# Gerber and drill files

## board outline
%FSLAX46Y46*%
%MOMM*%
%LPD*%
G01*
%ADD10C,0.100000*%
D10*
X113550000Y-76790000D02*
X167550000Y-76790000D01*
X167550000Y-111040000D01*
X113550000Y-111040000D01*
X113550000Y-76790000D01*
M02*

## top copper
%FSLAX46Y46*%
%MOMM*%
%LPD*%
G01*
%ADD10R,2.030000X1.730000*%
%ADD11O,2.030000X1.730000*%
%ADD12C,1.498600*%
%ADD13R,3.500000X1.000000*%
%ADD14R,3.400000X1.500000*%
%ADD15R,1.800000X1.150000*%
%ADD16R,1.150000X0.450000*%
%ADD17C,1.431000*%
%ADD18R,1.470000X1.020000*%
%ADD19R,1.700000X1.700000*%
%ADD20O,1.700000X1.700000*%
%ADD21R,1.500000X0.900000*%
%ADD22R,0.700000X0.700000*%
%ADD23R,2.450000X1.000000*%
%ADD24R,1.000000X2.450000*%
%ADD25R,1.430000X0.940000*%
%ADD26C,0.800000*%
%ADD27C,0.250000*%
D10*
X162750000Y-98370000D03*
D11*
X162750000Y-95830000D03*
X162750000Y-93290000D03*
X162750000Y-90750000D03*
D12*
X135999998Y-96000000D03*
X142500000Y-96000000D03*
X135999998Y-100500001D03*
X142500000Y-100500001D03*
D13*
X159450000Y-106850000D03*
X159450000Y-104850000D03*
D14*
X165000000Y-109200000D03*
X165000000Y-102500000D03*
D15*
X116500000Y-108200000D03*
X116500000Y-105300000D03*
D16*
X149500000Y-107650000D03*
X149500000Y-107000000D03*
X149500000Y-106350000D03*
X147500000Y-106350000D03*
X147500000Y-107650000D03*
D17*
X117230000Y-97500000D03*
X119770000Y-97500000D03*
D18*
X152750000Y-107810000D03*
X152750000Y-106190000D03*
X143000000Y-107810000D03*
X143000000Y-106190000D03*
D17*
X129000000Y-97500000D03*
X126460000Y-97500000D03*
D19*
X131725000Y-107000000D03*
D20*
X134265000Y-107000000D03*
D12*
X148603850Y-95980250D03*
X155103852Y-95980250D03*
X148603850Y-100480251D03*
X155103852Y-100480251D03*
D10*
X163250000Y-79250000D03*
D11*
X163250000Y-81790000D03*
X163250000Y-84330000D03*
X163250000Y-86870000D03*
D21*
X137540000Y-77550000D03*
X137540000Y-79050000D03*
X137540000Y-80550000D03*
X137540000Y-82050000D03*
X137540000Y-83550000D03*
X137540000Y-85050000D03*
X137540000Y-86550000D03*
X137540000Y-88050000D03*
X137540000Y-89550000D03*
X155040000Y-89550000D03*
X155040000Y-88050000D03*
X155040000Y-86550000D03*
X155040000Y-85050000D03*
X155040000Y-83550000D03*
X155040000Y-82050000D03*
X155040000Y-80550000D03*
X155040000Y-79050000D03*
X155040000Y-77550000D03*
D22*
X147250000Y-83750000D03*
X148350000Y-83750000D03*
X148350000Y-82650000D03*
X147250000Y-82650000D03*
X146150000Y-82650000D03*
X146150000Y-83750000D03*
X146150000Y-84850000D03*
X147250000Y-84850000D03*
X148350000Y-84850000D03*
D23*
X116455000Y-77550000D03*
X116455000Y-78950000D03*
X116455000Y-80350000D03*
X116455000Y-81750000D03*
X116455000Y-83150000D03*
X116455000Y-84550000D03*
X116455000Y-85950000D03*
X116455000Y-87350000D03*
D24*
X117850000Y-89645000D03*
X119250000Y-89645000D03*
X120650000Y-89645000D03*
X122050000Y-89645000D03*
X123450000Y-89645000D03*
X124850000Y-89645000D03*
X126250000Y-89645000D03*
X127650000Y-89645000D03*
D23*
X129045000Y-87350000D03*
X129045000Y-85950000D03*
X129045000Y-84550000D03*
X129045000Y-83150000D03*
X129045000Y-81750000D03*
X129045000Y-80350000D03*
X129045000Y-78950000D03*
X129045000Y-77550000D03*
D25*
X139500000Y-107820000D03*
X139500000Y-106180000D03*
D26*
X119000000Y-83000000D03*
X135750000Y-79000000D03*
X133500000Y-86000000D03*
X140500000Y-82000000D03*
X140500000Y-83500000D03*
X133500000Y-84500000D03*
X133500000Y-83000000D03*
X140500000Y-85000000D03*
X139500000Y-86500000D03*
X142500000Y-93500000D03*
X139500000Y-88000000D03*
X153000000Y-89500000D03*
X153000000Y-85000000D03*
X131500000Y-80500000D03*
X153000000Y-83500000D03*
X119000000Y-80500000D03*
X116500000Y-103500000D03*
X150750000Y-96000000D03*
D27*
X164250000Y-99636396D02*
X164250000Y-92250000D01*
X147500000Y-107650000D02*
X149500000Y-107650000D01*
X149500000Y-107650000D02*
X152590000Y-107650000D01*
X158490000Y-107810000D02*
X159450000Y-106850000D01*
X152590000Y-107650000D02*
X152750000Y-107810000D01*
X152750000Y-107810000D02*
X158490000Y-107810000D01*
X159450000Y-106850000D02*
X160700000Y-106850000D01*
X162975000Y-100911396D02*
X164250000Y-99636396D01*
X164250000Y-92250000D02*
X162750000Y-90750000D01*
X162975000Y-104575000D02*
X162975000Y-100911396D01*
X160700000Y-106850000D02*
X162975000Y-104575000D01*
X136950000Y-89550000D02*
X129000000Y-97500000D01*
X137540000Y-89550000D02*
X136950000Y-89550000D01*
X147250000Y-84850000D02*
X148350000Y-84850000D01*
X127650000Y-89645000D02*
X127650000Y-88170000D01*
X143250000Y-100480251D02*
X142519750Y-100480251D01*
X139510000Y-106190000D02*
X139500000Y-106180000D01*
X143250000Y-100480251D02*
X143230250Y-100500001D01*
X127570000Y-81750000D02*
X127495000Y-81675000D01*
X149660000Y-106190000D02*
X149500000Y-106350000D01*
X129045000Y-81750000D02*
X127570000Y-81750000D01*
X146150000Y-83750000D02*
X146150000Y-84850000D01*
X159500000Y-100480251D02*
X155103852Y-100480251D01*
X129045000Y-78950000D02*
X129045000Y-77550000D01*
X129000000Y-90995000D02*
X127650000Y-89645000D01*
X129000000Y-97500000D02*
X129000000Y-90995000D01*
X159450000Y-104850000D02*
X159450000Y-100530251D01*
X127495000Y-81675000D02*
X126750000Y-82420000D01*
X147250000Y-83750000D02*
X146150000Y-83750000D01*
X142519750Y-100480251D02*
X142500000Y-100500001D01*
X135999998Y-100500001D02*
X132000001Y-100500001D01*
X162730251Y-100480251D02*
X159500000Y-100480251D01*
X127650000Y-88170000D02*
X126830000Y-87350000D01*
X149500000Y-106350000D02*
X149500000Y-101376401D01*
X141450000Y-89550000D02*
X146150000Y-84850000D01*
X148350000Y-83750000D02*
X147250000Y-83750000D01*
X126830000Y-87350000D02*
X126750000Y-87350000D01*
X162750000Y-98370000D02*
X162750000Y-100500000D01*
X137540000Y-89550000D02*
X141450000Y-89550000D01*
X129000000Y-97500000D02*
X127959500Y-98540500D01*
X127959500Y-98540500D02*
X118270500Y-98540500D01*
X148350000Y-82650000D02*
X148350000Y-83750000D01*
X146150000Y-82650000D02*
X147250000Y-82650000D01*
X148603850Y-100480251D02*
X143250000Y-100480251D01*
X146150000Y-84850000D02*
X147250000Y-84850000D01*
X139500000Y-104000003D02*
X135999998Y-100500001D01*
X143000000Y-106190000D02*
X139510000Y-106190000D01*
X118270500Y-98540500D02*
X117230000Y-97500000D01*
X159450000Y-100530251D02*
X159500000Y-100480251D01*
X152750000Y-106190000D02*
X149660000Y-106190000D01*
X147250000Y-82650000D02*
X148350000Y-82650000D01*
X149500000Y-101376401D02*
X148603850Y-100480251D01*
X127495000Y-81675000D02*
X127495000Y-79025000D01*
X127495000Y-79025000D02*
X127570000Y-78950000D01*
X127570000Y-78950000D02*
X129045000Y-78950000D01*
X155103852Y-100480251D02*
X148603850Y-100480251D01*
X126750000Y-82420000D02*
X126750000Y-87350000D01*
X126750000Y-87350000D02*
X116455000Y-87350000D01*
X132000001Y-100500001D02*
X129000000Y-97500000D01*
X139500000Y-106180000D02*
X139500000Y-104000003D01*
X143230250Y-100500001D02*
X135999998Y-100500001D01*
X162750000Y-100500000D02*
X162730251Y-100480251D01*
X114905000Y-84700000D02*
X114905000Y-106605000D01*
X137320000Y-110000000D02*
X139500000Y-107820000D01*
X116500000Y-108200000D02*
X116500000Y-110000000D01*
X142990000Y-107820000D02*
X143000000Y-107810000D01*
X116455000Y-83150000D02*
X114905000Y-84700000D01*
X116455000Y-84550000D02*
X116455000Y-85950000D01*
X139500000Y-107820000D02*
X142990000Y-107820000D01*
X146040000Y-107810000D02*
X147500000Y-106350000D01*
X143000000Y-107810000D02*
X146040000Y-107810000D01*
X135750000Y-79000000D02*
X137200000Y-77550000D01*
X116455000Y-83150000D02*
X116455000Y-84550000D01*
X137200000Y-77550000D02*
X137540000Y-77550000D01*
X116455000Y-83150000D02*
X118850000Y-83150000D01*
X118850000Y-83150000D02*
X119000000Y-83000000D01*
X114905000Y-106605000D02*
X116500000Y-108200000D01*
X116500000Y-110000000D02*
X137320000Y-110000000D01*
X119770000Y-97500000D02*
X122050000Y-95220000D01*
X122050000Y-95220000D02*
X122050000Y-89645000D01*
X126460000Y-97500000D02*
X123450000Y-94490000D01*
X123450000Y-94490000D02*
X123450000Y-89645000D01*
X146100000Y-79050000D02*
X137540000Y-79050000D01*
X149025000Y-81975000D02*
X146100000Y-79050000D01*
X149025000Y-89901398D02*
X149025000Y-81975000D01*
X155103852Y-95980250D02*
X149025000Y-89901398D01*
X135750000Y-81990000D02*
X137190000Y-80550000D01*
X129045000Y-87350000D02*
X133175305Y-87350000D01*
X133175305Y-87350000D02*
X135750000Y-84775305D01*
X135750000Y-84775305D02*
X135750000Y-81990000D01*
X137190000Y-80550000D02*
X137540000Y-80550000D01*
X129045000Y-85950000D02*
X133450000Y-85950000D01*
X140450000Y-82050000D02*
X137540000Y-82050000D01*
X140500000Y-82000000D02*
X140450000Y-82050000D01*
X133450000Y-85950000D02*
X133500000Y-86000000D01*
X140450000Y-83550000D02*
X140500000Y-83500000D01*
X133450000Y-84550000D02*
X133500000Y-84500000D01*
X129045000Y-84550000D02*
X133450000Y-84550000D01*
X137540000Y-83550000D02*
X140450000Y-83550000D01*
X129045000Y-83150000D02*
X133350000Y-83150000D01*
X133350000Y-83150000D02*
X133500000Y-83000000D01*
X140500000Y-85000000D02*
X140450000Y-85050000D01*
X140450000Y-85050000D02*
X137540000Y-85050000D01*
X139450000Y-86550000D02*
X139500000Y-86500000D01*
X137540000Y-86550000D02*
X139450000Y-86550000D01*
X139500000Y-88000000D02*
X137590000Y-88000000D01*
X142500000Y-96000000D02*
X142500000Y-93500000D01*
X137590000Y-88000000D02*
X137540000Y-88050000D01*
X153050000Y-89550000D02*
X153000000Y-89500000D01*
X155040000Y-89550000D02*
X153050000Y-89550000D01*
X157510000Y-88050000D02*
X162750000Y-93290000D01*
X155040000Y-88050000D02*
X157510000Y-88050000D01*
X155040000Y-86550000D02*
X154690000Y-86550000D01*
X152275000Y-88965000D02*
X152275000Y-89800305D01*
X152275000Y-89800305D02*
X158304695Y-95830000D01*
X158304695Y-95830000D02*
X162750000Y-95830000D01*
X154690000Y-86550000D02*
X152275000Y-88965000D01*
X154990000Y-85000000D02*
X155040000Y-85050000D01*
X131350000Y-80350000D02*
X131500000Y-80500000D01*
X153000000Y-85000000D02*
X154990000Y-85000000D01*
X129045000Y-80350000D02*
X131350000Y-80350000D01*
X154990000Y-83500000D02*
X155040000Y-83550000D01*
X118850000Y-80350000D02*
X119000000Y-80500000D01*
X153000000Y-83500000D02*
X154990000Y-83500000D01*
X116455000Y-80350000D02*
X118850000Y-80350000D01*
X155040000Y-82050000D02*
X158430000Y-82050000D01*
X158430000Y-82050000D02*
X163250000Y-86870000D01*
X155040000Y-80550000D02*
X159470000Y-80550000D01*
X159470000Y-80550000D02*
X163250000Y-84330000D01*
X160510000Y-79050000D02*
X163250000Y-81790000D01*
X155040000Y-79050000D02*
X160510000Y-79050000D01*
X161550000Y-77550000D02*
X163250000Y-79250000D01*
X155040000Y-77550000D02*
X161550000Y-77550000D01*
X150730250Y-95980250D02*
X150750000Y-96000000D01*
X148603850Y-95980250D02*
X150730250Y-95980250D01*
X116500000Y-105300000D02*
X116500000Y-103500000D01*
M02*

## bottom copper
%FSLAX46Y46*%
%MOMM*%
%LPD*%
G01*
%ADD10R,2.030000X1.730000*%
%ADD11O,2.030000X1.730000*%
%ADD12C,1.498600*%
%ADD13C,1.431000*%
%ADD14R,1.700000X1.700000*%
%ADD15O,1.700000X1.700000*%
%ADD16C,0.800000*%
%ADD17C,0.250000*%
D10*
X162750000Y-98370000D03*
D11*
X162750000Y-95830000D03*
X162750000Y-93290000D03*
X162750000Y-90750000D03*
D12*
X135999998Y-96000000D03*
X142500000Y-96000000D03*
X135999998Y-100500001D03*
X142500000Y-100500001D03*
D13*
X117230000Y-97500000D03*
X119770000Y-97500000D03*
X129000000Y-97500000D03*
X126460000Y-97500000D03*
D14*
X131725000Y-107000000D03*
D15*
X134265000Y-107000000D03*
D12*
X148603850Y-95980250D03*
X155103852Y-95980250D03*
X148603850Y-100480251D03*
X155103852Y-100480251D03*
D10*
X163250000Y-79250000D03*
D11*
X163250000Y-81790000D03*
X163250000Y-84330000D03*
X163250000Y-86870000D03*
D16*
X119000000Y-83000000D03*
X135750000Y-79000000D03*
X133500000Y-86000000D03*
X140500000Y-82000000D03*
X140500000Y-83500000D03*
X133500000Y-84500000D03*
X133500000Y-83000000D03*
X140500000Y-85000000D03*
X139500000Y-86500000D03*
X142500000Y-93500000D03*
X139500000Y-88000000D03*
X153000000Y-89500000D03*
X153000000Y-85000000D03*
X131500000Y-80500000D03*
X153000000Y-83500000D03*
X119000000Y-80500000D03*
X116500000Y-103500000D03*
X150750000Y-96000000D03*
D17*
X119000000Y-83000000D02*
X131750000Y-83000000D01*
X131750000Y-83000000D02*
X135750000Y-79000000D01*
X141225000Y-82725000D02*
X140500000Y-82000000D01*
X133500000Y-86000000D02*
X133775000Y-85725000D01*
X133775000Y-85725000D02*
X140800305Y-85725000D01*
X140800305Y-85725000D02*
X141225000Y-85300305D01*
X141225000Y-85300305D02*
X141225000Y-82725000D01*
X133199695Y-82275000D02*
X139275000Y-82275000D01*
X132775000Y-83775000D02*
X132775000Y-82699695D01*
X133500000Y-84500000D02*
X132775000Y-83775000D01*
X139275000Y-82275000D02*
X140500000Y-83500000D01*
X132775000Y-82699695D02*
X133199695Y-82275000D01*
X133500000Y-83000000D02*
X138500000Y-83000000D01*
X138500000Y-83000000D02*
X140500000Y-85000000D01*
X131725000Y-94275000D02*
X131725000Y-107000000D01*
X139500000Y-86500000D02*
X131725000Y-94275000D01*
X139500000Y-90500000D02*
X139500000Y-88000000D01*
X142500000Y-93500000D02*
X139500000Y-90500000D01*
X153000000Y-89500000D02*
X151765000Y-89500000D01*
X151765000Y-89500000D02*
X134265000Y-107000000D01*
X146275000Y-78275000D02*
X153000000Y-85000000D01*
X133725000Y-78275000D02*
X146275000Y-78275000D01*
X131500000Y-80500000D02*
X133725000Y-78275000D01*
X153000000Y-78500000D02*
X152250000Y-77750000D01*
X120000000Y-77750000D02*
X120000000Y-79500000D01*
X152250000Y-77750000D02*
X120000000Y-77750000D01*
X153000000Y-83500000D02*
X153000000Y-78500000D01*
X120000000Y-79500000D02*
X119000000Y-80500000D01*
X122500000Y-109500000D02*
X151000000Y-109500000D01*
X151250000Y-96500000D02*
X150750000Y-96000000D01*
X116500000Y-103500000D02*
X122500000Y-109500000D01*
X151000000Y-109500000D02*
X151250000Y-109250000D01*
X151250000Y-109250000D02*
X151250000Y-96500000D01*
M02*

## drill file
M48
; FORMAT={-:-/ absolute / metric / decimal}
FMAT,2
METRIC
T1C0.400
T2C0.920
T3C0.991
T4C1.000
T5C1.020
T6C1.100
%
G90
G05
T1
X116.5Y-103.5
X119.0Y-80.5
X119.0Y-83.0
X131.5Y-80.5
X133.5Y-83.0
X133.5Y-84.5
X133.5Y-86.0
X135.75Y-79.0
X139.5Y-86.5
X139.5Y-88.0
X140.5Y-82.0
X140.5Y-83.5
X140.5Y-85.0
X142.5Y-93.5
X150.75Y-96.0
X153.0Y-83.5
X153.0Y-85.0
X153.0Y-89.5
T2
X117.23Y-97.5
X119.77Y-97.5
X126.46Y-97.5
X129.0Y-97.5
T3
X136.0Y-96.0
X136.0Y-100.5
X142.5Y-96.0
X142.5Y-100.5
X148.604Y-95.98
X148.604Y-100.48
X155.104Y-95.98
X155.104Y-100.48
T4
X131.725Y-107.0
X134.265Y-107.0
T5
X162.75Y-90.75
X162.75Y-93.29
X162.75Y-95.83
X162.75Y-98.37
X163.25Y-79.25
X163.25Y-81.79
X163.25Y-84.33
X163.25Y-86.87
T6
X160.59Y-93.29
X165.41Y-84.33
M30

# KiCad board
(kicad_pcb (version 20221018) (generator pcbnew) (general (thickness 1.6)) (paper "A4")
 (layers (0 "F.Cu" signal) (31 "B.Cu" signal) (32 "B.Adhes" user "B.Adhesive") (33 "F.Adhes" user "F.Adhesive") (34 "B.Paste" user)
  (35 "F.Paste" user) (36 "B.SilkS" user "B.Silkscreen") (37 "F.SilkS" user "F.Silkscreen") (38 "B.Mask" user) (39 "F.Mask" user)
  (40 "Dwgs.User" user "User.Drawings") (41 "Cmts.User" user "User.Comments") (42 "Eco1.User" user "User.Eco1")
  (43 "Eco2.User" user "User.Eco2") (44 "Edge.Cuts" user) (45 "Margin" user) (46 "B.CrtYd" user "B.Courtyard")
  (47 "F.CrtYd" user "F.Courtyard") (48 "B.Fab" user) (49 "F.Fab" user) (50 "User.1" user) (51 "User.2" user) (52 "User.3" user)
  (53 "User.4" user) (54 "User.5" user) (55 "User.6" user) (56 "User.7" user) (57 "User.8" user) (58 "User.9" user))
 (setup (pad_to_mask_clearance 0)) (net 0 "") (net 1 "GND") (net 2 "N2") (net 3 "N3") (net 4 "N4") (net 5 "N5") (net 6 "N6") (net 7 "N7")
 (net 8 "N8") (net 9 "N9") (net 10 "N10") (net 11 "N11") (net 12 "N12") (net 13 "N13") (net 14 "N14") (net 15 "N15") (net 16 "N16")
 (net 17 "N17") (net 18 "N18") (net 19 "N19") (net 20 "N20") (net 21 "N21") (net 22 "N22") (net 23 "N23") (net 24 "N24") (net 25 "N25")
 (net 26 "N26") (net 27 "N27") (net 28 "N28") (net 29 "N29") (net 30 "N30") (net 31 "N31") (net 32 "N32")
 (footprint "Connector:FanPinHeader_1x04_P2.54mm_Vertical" (layer "F.Cu") (at 162.75 98.37 90)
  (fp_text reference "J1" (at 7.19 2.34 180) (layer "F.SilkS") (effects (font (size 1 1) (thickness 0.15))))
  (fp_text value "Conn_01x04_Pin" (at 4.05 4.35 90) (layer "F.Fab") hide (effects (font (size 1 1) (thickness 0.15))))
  (pad "" np_thru_hole circle (at 5.08 -2.16 180) (size 1.1 1.1) (drill 1.1) (layers "*.Cu" "*.Mask"))
  (pad "1" thru_hole rect (at 0 0 180) (size 2.03 1.73) (drill 1.02) (layers "*.Cu" "*.Mask") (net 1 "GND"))
  (pad "2" thru_hole oval (at 2.54 0 180) (size 2.03 1.73) (drill 1.02) (layers "*.Cu" "*.Mask") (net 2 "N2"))
  (pad "3" thru_hole oval (at 5.08 0 180) (size 2.03 1.73) (drill 1.02) (layers "*.Cu" "*.Mask") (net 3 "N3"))
  (pad "4" thru_hole oval (at 7.62 0 180) (size 2.03 1.73) (drill 1.02) (layers "*.Cu" "*.Mask") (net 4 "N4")))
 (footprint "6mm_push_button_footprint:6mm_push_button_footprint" (layer "F.Cu") (at 135.999998 96)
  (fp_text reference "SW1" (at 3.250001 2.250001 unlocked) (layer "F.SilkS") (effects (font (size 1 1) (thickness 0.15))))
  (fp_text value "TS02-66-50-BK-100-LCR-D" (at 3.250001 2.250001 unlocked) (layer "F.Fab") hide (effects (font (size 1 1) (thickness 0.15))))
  (pad "1" thru_hole circle (at 0 0) (size 1.4986 1.4986) (drill 0.9906) (layers "*.Cu" "*.Mask") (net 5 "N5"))
  (pad "2" thru_hole circle (at 6.500002 0) (size 1.4986 1.4986) (drill 0.9906) (layers "*.Cu" "*.Mask") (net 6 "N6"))
  (pad "3" thru_hole circle (at 0 4.500001) (size 1.4986 1.4986) (drill 0.9906) (layers "*.Cu" "*.Mask") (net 1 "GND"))
  (pad "4" thru_hole circle (at 6.500002 4.500001) (size 1.4986 1.4986) (drill 0.9906) (layers "*.Cu" "*.Mask") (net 1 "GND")))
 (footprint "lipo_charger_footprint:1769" (layer "F.Cu") (at 159.45 105.85 90)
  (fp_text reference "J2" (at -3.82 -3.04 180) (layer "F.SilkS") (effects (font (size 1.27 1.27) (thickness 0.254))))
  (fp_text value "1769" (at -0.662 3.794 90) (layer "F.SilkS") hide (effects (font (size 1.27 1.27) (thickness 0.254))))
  (pad "1" smd rect (at -1 0 90) (size 1 3.5) (layers "F.Cu" "F.Paste" "F.Mask") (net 4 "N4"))
  (pad "2" smd rect (at 1 0 90) (size 1 3.5) (layers "F.Cu" "F.Paste" "F.Mask") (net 1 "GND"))
  (pad "3" smd rect (at -3.35 5.55 90) (size 1.5 3.4) (layers "F.Cu" "F.Paste" "F.Mask"))
  (pad "4" smd rect (at 3.35 5.55 90) (size 1.5 3.4) (layers "F.Cu" "F.Paste" "F.Mask")))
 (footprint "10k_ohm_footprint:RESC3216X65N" (layer "F.Cu") (at 116.5 106.75 90)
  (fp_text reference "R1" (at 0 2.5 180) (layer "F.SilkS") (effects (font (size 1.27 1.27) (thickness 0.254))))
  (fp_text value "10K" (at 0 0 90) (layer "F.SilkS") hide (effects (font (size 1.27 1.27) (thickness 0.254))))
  (pad "1" smd rect (at -1.45 0 90) (size 1.15 1.8) (layers "F.Cu" "F.Paste" "F.Mask") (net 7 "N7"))
  (pad "2" smd rect (at 1.45 0 90) (size 1.15 1.8) (layers "F.Cu" "F.Paste" "F.Mask") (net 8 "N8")))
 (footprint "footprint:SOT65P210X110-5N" (layer "F.Cu") (at 148.5 107 180)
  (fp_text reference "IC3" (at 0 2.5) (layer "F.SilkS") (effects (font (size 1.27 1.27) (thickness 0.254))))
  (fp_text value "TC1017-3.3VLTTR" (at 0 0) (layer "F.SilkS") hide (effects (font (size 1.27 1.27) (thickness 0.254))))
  (pad "1" smd rect (at -1 -0.65 270) (size 0.45 1.15) (layers "F.Cu" "F.Paste" "F.Mask") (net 4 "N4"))
  (pad "2" smd rect (at -1 0 270) (size 0.45 1.15) (layers "F.Cu" "F.Paste" "F.Mask") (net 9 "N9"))
  (pad "3" smd rect (at -1 0.65 270) (size 0.45 1.15) (layers "F.Cu" "F.Paste" "F.Mask") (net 1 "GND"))
  (pad "4" smd rect (at 1 0.65 270) (size 0.45 1.15) (layers "F.Cu" "F.Paste" "F.Mask") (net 7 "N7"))
  (pad "5" smd rect (at 1 -0.65 270) (size 0.45 1.15) (layers "F.Cu" "F.Paste" "F.Mask") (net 4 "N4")))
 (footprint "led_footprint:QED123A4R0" (layer "F.Cu") (at 117.23 97.5 180)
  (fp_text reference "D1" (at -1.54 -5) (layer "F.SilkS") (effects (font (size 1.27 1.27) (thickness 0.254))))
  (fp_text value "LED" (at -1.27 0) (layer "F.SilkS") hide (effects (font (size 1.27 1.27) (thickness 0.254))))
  (pad "1" thru_hole circle (at 0 0 180) (size 1.431 1.431) (drill 0.92) (layers "*.Cu" "*.Mask") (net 1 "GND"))
  (pad "2" thru_hole circle (at -2.54 0 180) (size 1.431 1.431) (drill 0.92) (layers "*.Cu" "*.Mask") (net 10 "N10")))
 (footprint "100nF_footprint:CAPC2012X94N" (layer "F.Cu") (at 152.75 107 90)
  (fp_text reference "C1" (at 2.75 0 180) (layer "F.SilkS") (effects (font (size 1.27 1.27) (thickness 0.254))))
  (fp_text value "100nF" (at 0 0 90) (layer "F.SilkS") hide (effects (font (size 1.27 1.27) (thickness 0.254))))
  (pad "1" smd rect (at -0.81 0 90) (size 1.02 1.47) (layers "F.Cu" "F.Paste" "F.Mask") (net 4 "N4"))
  (pad "2" smd rect (at 0.81 0 90) (size 1.02 1.47) (layers "F.Cu" "F.Paste" "F.Mask") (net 1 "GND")))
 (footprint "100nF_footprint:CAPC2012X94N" (layer "F.Cu") (at 143 107 90)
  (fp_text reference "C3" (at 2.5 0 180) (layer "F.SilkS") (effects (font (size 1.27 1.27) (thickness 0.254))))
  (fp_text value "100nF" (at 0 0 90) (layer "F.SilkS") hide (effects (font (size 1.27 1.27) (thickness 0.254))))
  (pad "1" smd rect (at -0.81 0 90) (size 1.02 1.47) (layers "F.Cu" "F.Paste" "F.Mask") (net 7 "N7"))
  (pad "2" smd rect (at 0.81 0 90) (size 1.02 1.47) (layers "F.Cu" "F.Paste" "F.Mask") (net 1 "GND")))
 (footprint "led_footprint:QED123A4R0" (layer "F.Cu") (at 129 97.5)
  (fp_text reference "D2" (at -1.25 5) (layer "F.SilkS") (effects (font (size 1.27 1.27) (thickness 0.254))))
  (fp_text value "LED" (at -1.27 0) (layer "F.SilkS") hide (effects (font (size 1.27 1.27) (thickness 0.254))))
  (pad "1" thru_hole circle (at 0 0) (size 1.431 1.431) (drill 0.92) (layers "*.Cu" "*.Mask") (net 1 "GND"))
  (pad "2" thru_hole circle (at -2.54 0) (size 1.431 1.431) (drill 0.92) (layers "*.Cu" "*.Mask") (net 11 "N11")))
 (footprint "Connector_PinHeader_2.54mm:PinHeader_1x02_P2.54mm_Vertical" (layer "F.Cu") (at 131.725 107 90)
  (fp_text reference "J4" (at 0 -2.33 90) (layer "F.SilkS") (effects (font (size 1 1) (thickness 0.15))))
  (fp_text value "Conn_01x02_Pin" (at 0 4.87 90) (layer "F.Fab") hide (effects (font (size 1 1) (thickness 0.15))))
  (pad "1" thru_hole rect (at 0 0 90) (size 1.7 1.7) (drill 1) (layers "*.Cu" "*.Mask") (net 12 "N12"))
  (pad "2" thru_hole oval (at 0 2.54 90) (size 1.7 1.7) (drill 1) (layers "*.Cu" "*.Mask") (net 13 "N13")))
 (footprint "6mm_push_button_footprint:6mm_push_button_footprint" (layer "F.Cu") (at 148.60385 95.98025)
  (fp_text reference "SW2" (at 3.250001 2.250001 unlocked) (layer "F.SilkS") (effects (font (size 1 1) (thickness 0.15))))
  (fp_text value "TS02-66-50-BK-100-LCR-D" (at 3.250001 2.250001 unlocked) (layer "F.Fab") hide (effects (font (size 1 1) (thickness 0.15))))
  (pad "1" thru_hole circle (at 0 0) (size 1.4986 1.4986) (drill 0.9906) (layers "*.Cu" "*.Mask") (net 8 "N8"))
  (pad "2" thru_hole circle (at 6.500002 0) (size 1.4986 1.4986) (drill 0.9906) (layers "*.Cu" "*.Mask") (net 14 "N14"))
  (pad "3" thru_hole circle (at 0 4.500001) (size 1.4986 1.4986) (drill 0.9906) (layers "*.Cu" "*.Mask") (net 1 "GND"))
  (pad "4" thru_hole circle (at 6.500002 4.500001) (size 1.4986 1.4986) (drill 0.9906) (layers "*.Cu" "*.Mask") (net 1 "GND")))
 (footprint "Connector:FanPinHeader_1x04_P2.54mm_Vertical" (layer "F.Cu") (at 163.25 79.25 -90)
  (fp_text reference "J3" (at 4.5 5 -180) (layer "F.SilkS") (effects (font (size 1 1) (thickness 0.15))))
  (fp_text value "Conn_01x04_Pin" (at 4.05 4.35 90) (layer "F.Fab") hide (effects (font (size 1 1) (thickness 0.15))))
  (pad "" np_thru_hole circle (at 5.08 -2.16) (size 1.1 1.1) (drill 1.1) (layers "*.Cu" "*.Mask"))
  (pad "1" thru_hole rect (at 0 0) (size 2.03 1.73) (drill 1.02) (layers "*.Cu" "*.Mask") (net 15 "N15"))
  (pad "2" thru_hole oval (at 2.54 0) (size 2.03 1.73) (drill 1.02) (layers "*.Cu" "*.Mask") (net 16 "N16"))
  (pad "3" thru_hole oval (at 5.08 0) (size 2.03 1.73) (drill 1.02) (layers "*.Cu" "*.Mask") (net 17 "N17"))
  (pad "4" thru_hole oval (at 7.62 0) (size 2.03 1.73) (drill 1.02) (layers "*.Cu" "*.Mask") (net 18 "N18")))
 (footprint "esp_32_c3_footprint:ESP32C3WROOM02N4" (layer "F.Cu") (at 147.25 83.75)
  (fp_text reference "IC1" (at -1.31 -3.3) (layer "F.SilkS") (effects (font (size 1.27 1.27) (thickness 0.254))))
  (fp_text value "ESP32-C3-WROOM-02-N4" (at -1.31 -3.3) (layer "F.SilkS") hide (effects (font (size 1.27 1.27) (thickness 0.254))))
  (pad "1" smd rect (at -9.71 -6.2 90) (size 0.9 1.5) (layers "F.Cu" "F.Paste" "F.Mask") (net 7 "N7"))
  (pad "2" smd rect (at -9.71 -4.7 90) (size 0.9 1.5) (layers "F.Cu" "F.Paste" "F.Mask") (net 14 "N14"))
  (pad "3" smd rect (at -9.71 -3.2 90) (size 0.9 1.5) (layers "F.Cu" "F.Paste" "F.Mask") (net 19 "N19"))
  (pad "4" smd rect (at -9.71 -1.7 90) (size 0.9 1.5) (layers "F.Cu" "F.Paste" "F.Mask") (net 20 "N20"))
  (pad "5" smd rect (at -9.71 -0.2 90) (size 0.9 1.5) (layers "F.Cu" "F.Paste" "F.Mask") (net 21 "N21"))
  (pad "6" smd rect (at -9.71 1.3 90) (size 0.9 1.5) (layers "F.Cu" "F.Paste" "F.Mask") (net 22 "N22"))
  (pad "7" smd rect (at -9.71 2.8 90) (size 0.9 1.5) (layers "F.Cu" "F.Paste" "F.Mask") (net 12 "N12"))
  (pad "8" smd rect (at -9.71 4.3 90) (size 0.9 1.5) (layers "F.Cu" "F.Paste" "F.Mask") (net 6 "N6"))
  (pad "9" smd rect (at -9.71 5.8 90) (size 0.9 1.5) (layers "F.Cu" "F.Paste" "F.Mask") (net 1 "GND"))
  (pad "10" smd rect (at 7.79 5.8 90) (size 0.9 1.5) (layers "F.Cu" "F.Paste" "F.Mask") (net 13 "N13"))
  (pad "11" smd rect (at 7.79 4.3 90) (size 0.9 1.5) (layers "F.Cu" "F.Paste" "F.Mask") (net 3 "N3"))
  (pad "12" smd rect (at 7.79 2.8 90) (size 0.9 1.5) (layers "F.Cu" "F.Paste" "F.Mask") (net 2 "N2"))
  (pad "13" smd rect (at 7.79 1.3 90) (size 0.9 1.5) (layers "F.Cu" "F.Paste" "F.Mask") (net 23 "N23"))
  (pad "14" smd rect (at 7.79 -0.2 90) (size 0.9 1.5) (layers "F.Cu" "F.Paste" "F.Mask") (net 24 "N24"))
  (pad "15" smd rect (at 7.79 -1.7 90) (size 0.9 1.5) (layers "F.Cu" "F.Paste" "F.Mask") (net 18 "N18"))
  (pad "16" smd rect (at 7.79 -3.2 90) (size 0.9 1.5) (layers "F.Cu" "F.Paste" "F.Mask") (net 17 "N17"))
  (pad "17" smd rect (at 7.79 -4.7 90) (size 0.9 1.5) (layers "F.Cu" "F.Paste" "F.Mask") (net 16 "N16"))
  (pad "18" smd rect (at 7.79 -6.2 90) (size 0.9 1.5) (layers "F.Cu" "F.Paste" "F.Mask") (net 15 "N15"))
  (pad "19" smd rect (at 0 0 90) (size 0.7 0.7) (layers "F.Cu" "F.Paste" "F.Mask") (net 1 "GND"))
  (pad "20" smd rect (at 1.1 0 90) (size 0.7 0.7) (layers "F.Cu" "F.Paste" "F.Mask") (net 1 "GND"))
  (pad "21" smd rect (at 1.1 -1.1 90) (size 0.7 0.7) (layers "F.Cu" "F.Paste" "F.Mask") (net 1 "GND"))
  (pad "22" smd rect (at 0 -1.1 90) (size 0.7 0.7) (layers "F.Cu" "F.Paste" "F.Mask") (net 1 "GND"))
  (pad "23" smd rect (at -1.1 -1.1 90) (size 0.7 0.7) (layers "F.Cu" "F.Paste" "F.Mask") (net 1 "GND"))
  (pad "24" smd rect (at -1.1 0 90) (size 0.7 0.7) (layers "F.Cu" "F.Paste" "F.Mask") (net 1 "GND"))
  (pad "25" smd rect (at -1.1 1.1 90) (size 0.7 0.7) (layers "F.Cu" "F.Paste" "F.Mask") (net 1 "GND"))
  (pad "26" smd rect (at 0 1.1 90) (size 0.7 0.7) (layers "F.Cu" "F.Paste" "F.Mask") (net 1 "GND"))
  (pad "27" smd rect (at 1.1 1.1 90) (size 0.7 0.7) (layers "F.Cu" "F.Paste" "F.Mask") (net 1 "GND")))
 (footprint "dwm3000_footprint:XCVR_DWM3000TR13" (layer "F.Cu") (at 122.75 78.5)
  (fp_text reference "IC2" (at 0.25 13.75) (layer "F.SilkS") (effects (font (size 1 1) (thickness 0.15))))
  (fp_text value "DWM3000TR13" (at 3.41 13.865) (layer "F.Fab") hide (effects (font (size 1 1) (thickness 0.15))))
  (pad "1" smd rect (at -6.295 -0.95) (size 2.45 1) (layers "F.Cu" "F.Paste" "F.Mask") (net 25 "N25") (solder_mask_margin 0.102))
  (pad "2" smd rect (at -6.295 0.45) (size 2.45 1) (layers "F.Cu" "F.Paste" "F.Mask") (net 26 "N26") (solder_mask_margin 0.102))
  (pad "3" smd rect (at -6.295 1.85) (size 2.45 1) (layers "F.Cu" "F.Paste" "F.Mask") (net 24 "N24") (solder_mask_margin 0.102))
  (pad "4" smd rect (at -6.295 3.25) (size 2.45 1) (layers "F.Cu" "F.Paste" "F.Mask") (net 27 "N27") (solder_mask_margin 0.102))
  (pad "5" smd rect (at -6.295 4.65) (size 2.45 1) (layers "F.Cu" "F.Paste" "F.Mask") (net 7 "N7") (solder_mask_margin 0.102))
  (pad "6" smd rect (at -6.295 6.05) (size 2.45 1) (layers "F.Cu" "F.Paste" "F.Mask") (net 7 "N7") (solder_mask_margin 0.102))
  (pad "7" smd rect (at -6.295 7.45) (size 2.45 1) (layers "F.Cu" "F.Paste" "F.Mask") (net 7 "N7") (solder_mask_margin 0.102))
  (pad "8" smd rect (at -6.295 8.85) (size 2.45 1) (layers "F.Cu" "F.Paste" "F.Mask") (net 1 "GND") (solder_mask_margin 0.102))
  (pad "9" smd rect (at -4.9 11.145) (size 1 2.45) (layers "F.Cu" "F.Paste" "F.Mask") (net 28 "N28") (solder_mask_margin 0.102))
  (pad "10" smd rect (at -3.5 11.145) (size 1 2.45) (layers "F.Cu" "F.Paste" "F.Mask") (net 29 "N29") (solder_mask_margin 0.102))
  (pad "11" smd rect (at -2.1 11.145) (size 1 2.45) (layers "F.Cu" "F.Paste" "F.Mask") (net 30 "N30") (solder_mask_margin 0.102))
  (pad "12" smd rect (at -0.7 11.145) (size 1 2.45) (layers "F.Cu" "F.Paste" "F.Mask") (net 10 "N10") (solder_mask_margin 0.102))
  (pad "13" smd rect (at 0.7 11.145) (size 1 2.45) (layers "F.Cu" "F.Paste" "F.Mask") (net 11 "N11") (solder_mask_margin 0.102))
  (pad "14" smd rect (at 2.1 11.145) (size 1 2.45) (layers "F.Cu" "F.Paste" "F.Mask") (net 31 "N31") (solder_mask_margin 0.102))
  (pad "15" smd rect (at 3.5 11.145) (size 1 2.45) (layers "F.Cu" "F.Paste" "F.Mask") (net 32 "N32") (solder_mask_margin 0.102))
  (pad "16" smd rect (at 4.9 11.145) (size 1 2.45) (layers "F.Cu" "F.Paste" "F.Mask") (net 1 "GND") (solder_mask_margin 0.102))
  (pad "17" smd rect (at 6.295 8.85) (size 2.45 1) (layers "F.Cu" "F.Paste" "F.Mask") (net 19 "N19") (solder_mask_margin 0.102))
  (pad "18" smd rect (at 6.295 7.45) (size 2.45 1) (layers "F.Cu" "F.Paste" "F.Mask") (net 20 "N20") (solder_mask_margin 0.102))
  (pad "19" smd rect (at 6.295 6.05) (size 2.45 1) (layers "F.Cu" "F.Paste" "F.Mask") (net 21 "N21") (solder_mask_margin 0.102))
  (pad "20" smd rect (at 6.295 4.65) (size 2.45 1) (layers "F.Cu" "F.Paste" "F.Mask") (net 22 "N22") (solder_mask_margin 0.102))
  (pad "21" smd rect (at 6.295 3.25) (size 2.45 1) (layers "F.Cu" "F.Paste" "F.Mask") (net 1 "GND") (solder_mask_margin 0.102))
  (pad "22" smd rect (at 6.295 1.85) (size 2.45 1) (layers "F.Cu" "F.Paste" "F.Mask") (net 23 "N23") (solder_mask_margin 0.102))
  (pad "23" smd rect (at 6.295 0.45) (size 2.45 1) (layers "F.Cu" "F.Paste" "F.Mask") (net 1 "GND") (solder_mask_margin 0.102))
  (pad "24" smd rect (at 6.295 -0.95) (size 2.45 1) (layers "F.Cu" "F.Paste" "F.Mask") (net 1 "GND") (solder_mask_margin 0.102))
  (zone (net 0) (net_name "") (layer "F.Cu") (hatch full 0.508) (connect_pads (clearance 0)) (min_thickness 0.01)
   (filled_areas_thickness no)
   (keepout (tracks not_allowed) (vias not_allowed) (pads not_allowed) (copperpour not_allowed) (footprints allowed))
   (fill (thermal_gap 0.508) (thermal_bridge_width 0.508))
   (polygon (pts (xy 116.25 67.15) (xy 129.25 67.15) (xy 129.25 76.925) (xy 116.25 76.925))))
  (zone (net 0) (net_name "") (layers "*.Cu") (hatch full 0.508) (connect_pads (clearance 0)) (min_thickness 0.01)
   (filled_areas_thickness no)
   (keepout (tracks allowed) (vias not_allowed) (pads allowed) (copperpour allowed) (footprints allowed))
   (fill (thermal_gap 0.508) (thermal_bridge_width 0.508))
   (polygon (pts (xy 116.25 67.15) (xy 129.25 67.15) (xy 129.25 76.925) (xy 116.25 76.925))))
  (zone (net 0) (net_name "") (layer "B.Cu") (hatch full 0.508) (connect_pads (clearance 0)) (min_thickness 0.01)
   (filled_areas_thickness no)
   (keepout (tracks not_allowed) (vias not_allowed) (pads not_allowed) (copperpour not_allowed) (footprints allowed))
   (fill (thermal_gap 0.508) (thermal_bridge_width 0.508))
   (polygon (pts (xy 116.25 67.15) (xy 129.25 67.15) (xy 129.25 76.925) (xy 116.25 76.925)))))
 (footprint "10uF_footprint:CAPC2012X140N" (layer "F.Cu") (at 139.5 107 90)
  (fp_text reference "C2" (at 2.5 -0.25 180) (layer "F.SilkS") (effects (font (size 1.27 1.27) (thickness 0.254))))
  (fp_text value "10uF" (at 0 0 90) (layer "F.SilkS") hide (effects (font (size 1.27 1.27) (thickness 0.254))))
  (pad "1" smd rect (at -0.82 0 90) (size 0.94 1.43) (layers "F.Cu" "F.Paste" "F.Mask") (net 7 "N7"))
  (pad "2" smd rect (at 0.82 0 90) (size 0.94 1.43) (layers "F.Cu" "F.Paste" "F.Mask") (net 1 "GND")))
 (gr_rect (start 113.55 76.79) (end 167.55 111.04) (stroke (width 0.1) (type default)) (fill none) (layer "Edge.Cuts"))
 (segment (start 164.25 99.636396) (end 164.25 92.25) (width 0.25) (layer "F.Cu") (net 4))
 (segment (start 147.5 107.65) (end 149.5 107.65) (width 0.25) (layer "F.Cu") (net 4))
 (segment (start 149.5 107.65) (end 152.59 107.65) (width 0.25) (layer "F.Cu") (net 4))
 (segment (start 158.49 107.81) (end 159.45 106.85) (width 0.25) (layer "F.Cu") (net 4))
 (segment (start 152.59 107.65) (end 152.75 107.81) (width 0.25) (layer "F.Cu") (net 4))
 (segment (start 152.75 107.81) (end 158.49 107.81) (width 0.25) (layer "F.Cu") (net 4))
 (segment (start 159.45 106.85) (end 160.7 106.85) (width 0.25) (layer "F.Cu") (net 4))
 (segment (start 162.975 100.911396) (end 164.25 99.636396) (width 0.25) (layer "F.Cu") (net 4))
 (segment (start 164.25 92.25) (end 162.75 90.75) (width 0.25) (layer "F.Cu") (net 4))
 (segment (start 162.975 104.575) (end 162.975 100.911396) (width 0.25) (layer "F.Cu") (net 4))
 (segment (start 160.7 106.85) (end 162.975 104.575) (width 0.25) (layer "F.Cu") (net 4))
 (segment (start 136.95 89.55) (end 129 97.5) (width 0.25) (layer "F.Cu") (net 1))
 (segment (start 137.54 89.55) (end 136.95 89.55) (width 0.25) (layer "F.Cu") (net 1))
 (segment (start 147.25 84.85) (end 148.35 84.85) (width 0.25) (layer "F.Cu") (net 1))
 (segment (start 127.65 89.645) (end 127.65 88.17) (width 0.25) (layer "F.Cu") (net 1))
 (segment (start 143.25 100.480251) (end 142.51975 100.480251) (width 0.25) (layer "F.Cu") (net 1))
 (segment (start 139.51 106.19) (end 139.5 106.18) (width 0.25) (layer "F.Cu") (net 1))
 (segment (start 143.25 100.480251) (end 143.23025 100.500001) (width 0.25) (layer "F.Cu") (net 1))
 (segment (start 127.57 81.75) (end 127.495 81.675) (width 0.25) (layer "F.Cu") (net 1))
 (segment (start 149.66 106.19) (end 149.5 106.35) (width 0.25) (layer "F.Cu") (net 1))
 (segment (start 129.045 81.75) (end 127.57 81.75) (width 0.25) (layer "F.Cu") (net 1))
 (segment (start 146.15 83.75) (end 146.15 84.85) (width 0.25) (layer "F.Cu") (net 1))
 (segment (start 159.5 100.480251) (end 155.103852 100.480251) (width 0.25) (layer "F.Cu") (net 1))
 (segment (start 129.045 78.95) (end 129.045 77.55) (width 0.25) (layer "F.Cu") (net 1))
 (segment (start 129 90.995) (end 127.65 89.645) (width 0.25) (layer "F.Cu") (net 1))
 (segment (start 129 97.5) (end 129 90.995) (width 0.25) (layer "F.Cu") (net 1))
 (segment (start 159.45 104.85) (end 159.45 100.530251) (width 0.25) (layer "F.Cu") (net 1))
 (segment (start 127.495 81.675) (end 126.75 82.42) (width 0.25) (layer "F.Cu") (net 1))
 (segment (start 147.25 83.75) (end 146.15 83.75) (width 0.25) (layer "F.Cu") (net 1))
 (segment (start 142.51975 100.480251) (end 142.5 100.500001) (width 0.25) (layer "F.Cu") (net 1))
 (segment (start 135.999998 100.500001) (end 132.000001 100.500001) (width 0.25) (layer "F.Cu") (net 1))
 (segment (start 162.730251 100.480251) (end 159.5 100.480251) (width 0.25) (layer "F.Cu") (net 1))
 (segment (start 127.65 88.17) (end 126.83 87.35) (width 0.25) (layer "F.Cu") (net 1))
 (segment (start 149.5 106.35) (end 149.5 101.376401) (width 0.25) (layer "F.Cu") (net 1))
 (segment (start 141.45 89.55) (end 146.15 84.85) (width 0.25) (layer "F.Cu") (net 1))
 (segment (start 148.35 83.75) (end 147.25 83.75) (width 0.25) (layer "F.Cu") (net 1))
 (segment (start 126.83 87.35) (end 126.75 87.35) (width 0.25) (layer "F.Cu") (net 1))
 (segment (start 162.75 98.37) (end 162.75 100.5) (width 0.25) (layer "F.Cu") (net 1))
 (segment (start 137.54 89.55) (end 141.45 89.55) (width 0.25) (layer "F.Cu") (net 1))
 (segment (start 129 97.5) (end 127.9595 98.5405) (width 0.25) (layer "F.Cu") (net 1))
 (segment (start 127.9595 98.5405) (end 118.2705 98.5405) (width 0.25) (layer "F.Cu") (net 1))
 (segment (start 148.35 82.65) (end 148.35 83.75) (width 0.25) (layer "F.Cu") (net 1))
 (segment (start 146.15 82.65) (end 147.25 82.65) (width 0.25) (layer "F.Cu") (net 1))
 (segment (start 148.60385 100.480251) (end 143.25 100.480251) (width 0.25) (layer "F.Cu") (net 1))
 (segment (start 146.15 84.85) (end 147.25 84.85) (width 0.25) (layer "F.Cu") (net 1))
 (segment (start 139.5 104.000003) (end 135.999998 100.500001) (width 0.25) (layer "F.Cu") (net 1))
 (segment (start 143 106.19) (end 139.51 106.19) (width 0.25) (layer "F.Cu") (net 1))
 (segment (start 118.2705 98.5405) (end 117.23 97.5) (width 0.25) (layer "F.Cu") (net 1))
 (segment (start 159.45 100.530251) (end 159.5 100.480251) (width 0.25) (layer "F.Cu") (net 1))
 (segment (start 152.75 106.19) (end 149.66 106.19) (width 0.25) (layer "F.Cu") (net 1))
 (segment (start 147.25 82.65) (end 148.35 82.65) (width 0.25) (layer "F.Cu") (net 1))
 (segment (start 149.5 101.376401) (end 148.60385 100.480251) (width 0.25) (layer "F.Cu") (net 1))
 (segment (start 127.495 81.675) (end 127.495 79.025) (width 0.25) (layer "F.Cu") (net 1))
 (segment (start 127.495 79.025) (end 127.57 78.95) (width 0.25) (layer "F.Cu") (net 1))
 (segment (start 127.57 78.95) (end 129.045 78.95) (width 0.25) (layer "F.Cu") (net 1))
 (segment (start 155.103852 100.480251) (end 148.60385 100.480251) (width 0.25) (layer "F.Cu") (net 1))
 (segment (start 126.75 82.42) (end 126.75 87.35) (width 0.25) (layer "F.Cu") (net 1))
 (segment (start 126.75 87.35) (end 116.455 87.35) (width 0.25) (layer "F.Cu") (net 1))
 (segment (start 132.000001 100.500001) (end 129 97.5) (width 0.25) (layer "F.Cu") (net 1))
 (segment (start 139.5 106.18) (end 139.5 104.000003) (width 0.25) (layer "F.Cu") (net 1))
 (segment (start 143.23025 100.500001) (end 135.999998 100.500001) (width 0.25) (layer "F.Cu") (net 1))
 (segment (start 162.75 100.5) (end 162.730251 100.480251) (width 0.25) (layer "F.Cu") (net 1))
 (segment (start 114.905 84.7) (end 114.905 106.605) (width 0.25) (layer "F.Cu") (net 7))
 (segment (start 137.32 110) (end 139.5 107.82) (width 0.25) (layer "F.Cu") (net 7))
 (segment (start 116.5 108.2) (end 116.5 110) (width 0.25) (layer "F.Cu") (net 7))
 (segment (start 142.99 107.82) (end 143 107.81) (width 0.25) (layer "F.Cu") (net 7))
 (segment (start 116.455 83.15) (end 114.905 84.7) (width 0.25) (layer "F.Cu") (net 7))
 (segment (start 116.455 84.55) (end 116.455 85.95) (width 0.25) (layer "F.Cu") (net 7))
 (segment (start 139.5 107.82) (end 142.99 107.82) (width 0.25) (layer "F.Cu") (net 7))
 (segment (start 146.04 107.81) (end 147.5 106.35) (width 0.25) (layer "F.Cu") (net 7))
 (segment (start 143 107.81) (end 146.04 107.81) (width 0.25) (layer "F.Cu") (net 7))
 (segment (start 135.75 79) (end 137.2 77.55) (width 0.25) (layer "F.Cu") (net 7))
 (segment (start 116.455 83.15) (end 116.455 84.55) (width 0.25) (layer "F.Cu") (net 7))
 (segment (start 137.2 77.55) (end 137.54 77.55) (width 0.25) (layer "F.Cu") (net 7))
 (segment (start 116.455 83.15) (end 118.85 83.15) (width 0.25) (layer "F.Cu") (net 7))
 (segment (start 118.85 83.15) (end 119 83) (width 0.25) (layer "F.Cu") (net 7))
 (segment (start 114.905 106.605) (end 116.5 108.2) (width 0.25) (layer "F.Cu") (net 7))
 (segment (start 116.5 110) (end 137.32 110) (width 0.25) (layer "F.Cu") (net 7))
 (via blind (at 119 83) (size 0.8) (drill 0.4) (layers "F.Cu" "B.Cu") (free) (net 7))
 (via blind (at 135.75 79) (size 0.8) (drill 0.4) (layers "F.Cu" "B.Cu") (free) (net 7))
 (segment (start 119 83) (end 131.75 83) (width 0.25) (layer "B.Cu") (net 7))
 (segment (start 131.75 83) (end 135.75 79) (width 0.25) (layer "B.Cu") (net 7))
 (segment (start 119.77 97.5) (end 122.05 95.22) (width 0.25) (layer "F.Cu") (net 10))
 (segment (start 122.05 95.22) (end 122.05 89.645) (width 0.25) (layer "F.Cu") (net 10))
 (segment (start 126.46 97.5) (end 123.45 94.49) (width 0.25) (layer "F.Cu") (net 11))
 (segment (start 123.45 94.49) (end 123.45 89.645) (width 0.25) (layer "F.Cu") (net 11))
 (segment (start 146.1 79.05) (end 137.54 79.05) (width 0.25) (layer "F.Cu") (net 14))
 (segment (start 149.025 81.975) (end 146.1 79.05) (width 0.25) (layer "F.Cu") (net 14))
 (segment (start 149.025 89.901398) (end 149.025 81.975) (width 0.25) (layer "F.Cu") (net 14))
 (segment (start 155.103852 95.98025) (end 149.025 89.901398) (width 0.25) (layer "F.Cu") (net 14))
 (segment (start 135.75 81.99) (end 137.19 80.55) (width 0.25) (layer "F.Cu") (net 19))
 (segment (start 129.045 87.35) (end 133.175305 87.35) (width 0.25) (layer "F.Cu") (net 19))
 (segment (start 133.175305 87.35) (end 135.75 84.775305) (width 0.25) (layer "F.Cu") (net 19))
 (segment (start 135.75 84.775305) (end 135.75 81.99) (width 0.25) (layer "F.Cu") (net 19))
 (segment (start 137.19 80.55) (end 137.54 80.55) (width 0.25) (layer "F.Cu") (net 19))
 (segment (start 129.045 85.95) (end 133.45 85.95) (width 0.25) (layer "F.Cu") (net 20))
 (segment (start 140.45 82.05) (end 137.54 82.05) (width 0.25) (layer "F.Cu") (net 20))
 (segment (start 140.5 82) (end 140.45 82.05) (width 0.25) (layer "F.Cu") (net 20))
 (segment (start 133.45 85.95) (end 133.5 86) (width 0.25) (layer "F.Cu") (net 20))
 (via blind (at 133.5 86) (size 0.8) (drill 0.4) (layers "F.Cu" "B.Cu") (free) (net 20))
 (via blind (at 140.5 82) (size 0.8) (drill 0.4) (layers "F.Cu" "B.Cu") (free) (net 20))
 (segment (start 141.225 82.725) (end 140.5 82) (width 0.25) (layer "B.Cu") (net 20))
 (segment (start 133.5 86) (end 133.775 85.725) (width 0.25) (layer "B.Cu") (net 20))
 (segment (start 133.775 85.725) (end 140.800305 85.725) (width 0.25) (layer "B.Cu") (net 20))
 (segment (start 140.800305 85.725) (end 141.225 85.300305) (width 0.25) (layer "B.Cu") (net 20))
 (segment (start 141.225 85.300305) (end 141.225 82.725) (width 0.25) (layer "B.Cu") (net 20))
 (segment (start 140.45 83.55) (end 140.5 83.5) (width 0.25) (layer "F.Cu") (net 21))
 (segment (start 133.45 84.55) (end 133.5 84.5) (width 0.25) (layer "F.Cu") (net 21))
 (segment (start 129.045 84.55) (end 133.45 84.55) (width 0.25) (layer "F.Cu") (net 21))
 (segment (start 137.54 83.55) (end 140.45 83.55) (width 0.25) (layer "F.Cu") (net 21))
 (via blind (at 140.5 83.5) (size 0.8) (drill 0.4) (layers "F.Cu" "B.Cu") (free) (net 21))
 (via blind (at 133.5 84.5) (size 0.8) (drill 0.4) (layers "F.Cu" "B.Cu") (free) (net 21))
 (segment (start 133.199695 82.275) (end 139.275 82.275) (width 0.25) (layer "B.Cu") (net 21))
 (segment (start 132.775 83.775) (end 132.775 82.699695) (width 0.25) (layer "B.Cu") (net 21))
 (segment (start 133.5 84.5) (end 132.775 83.775) (width 0.25) (layer "B.Cu") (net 21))
 (segment (start 139.275 82.275) (end 140.5 83.5) (width 0.25) (layer "B.Cu") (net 21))
 (segment (start 132.775 82.699695) (end 133.199695 82.275) (width 0.25) (layer "B.Cu") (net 21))
 (segment (start 129.045 83.15) (end 133.35 83.15) (width 0.25) (layer "F.Cu") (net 22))
 (segment (start 133.35 83.15) (end 133.5 83) (width 0.25) (layer "F.Cu") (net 22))
 (segment (start 140.5 85) (end 140.45 85.05) (width 0.25) (layer "F.Cu") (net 22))
 (segment (start 140.45 85.05) (end 137.54 85.05) (width 0.25) (layer "F.Cu") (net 22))
 (via blind (at 133.5 83) (size 0.8) (drill 0.4) (layers "F.Cu" "B.Cu") (free) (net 22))
 (via blind (at 140.5 85) (size 0.8) (drill 0.4) (layers "F.Cu" "B.Cu") (free) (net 22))
 (segment (start 133.5 83) (end 138.5 83) (width 0.25) (layer "B.Cu") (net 22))
 (segment (start 138.5 83) (end 140.5 85) (width 0.25) (layer "B.Cu") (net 22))
 (segment (start 139.45 86.55) (end 139.5 86.5) (width 0.25) (layer "F.Cu") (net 12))
 (segment (start 137.54 86.55) (end 139.45 86.55) (width 0.25) (layer "F.Cu") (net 12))
 (via blind (at 139.5 86.5) (size 0.8) (drill 0.4) (layers "F.Cu" "B.Cu") (free) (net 12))
 (segment (start 131.725 94.275) (end 131.725 107) (width 0.25) (layer "B.Cu") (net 12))
 (segment (start 139.5 86.5) (end 131.725 94.275) (width 0.25) (layer "B.Cu") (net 12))
 (segment (start 139.5 88) (end 137.59 88) (width 0.25) (layer "F.Cu") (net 6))
 (segment (start 142.5 96) (end 142.5 93.5) (width 0.25) (layer "F.Cu") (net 6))
 (segment (start 137.59 88) (end 137.54 88.05) (width 0.25) (layer "F.Cu") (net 6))
 (via blind (at 142.5 93.5) (size 0.8) (drill 0.4) (layers "F.Cu" "B.Cu") (free) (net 6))
 (via blind (at 139.5 88) (size 0.8) (drill 0.4) (layers "F.Cu" "B.Cu") (free) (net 6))
 (segment (start 139.5 90.5) (end 139.5 88) (width 0.25) (layer "B.Cu") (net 6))
 (segment (start 142.5 93.5) (end 139.5 90.5) (width 0.25) (layer "B.Cu") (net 6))
 (segment (start 153.05 89.55) (end 153 89.5) (width 0.25) (layer "F.Cu") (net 13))
 (segment (start 155.04 89.55) (end 153.05 89.55) (width 0.25) (layer "F.Cu") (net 13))
 (via blind (at 153 89.5) (size 0.8) (drill 0.4) (layers "F.Cu" "B.Cu") (free) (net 13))
 (segment (start 153 89.5) (end 151.765 89.5) (width 0.25) (layer "B.Cu") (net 13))
 (segment (start 151.765 89.5) (end 134.265 107) (width 0.25) (layer "B.Cu") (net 13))
 (segment (start 157.51 88.05) (end 162.75 93.29) (width 0.25) (layer "F.Cu") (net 3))
 (segment (start 155.04 88.05) (end 157.51 88.05) (width 0.25) (layer "F.Cu") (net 3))
 (segment (start 155.04 86.55) (end 154.69 86.55) (width 0.25) (layer "F.Cu") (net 2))
 (segment (start 152.275 88.965) (end 152.275 89.800305) (width 0.25) (layer "F.Cu") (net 2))
 (segment (start 152.275 89.800305) (end 158.304695 95.83) (width 0.25) (layer "F.Cu") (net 2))
 (segment (start 158.304695 95.83) (end 162.75 95.83) (width 0.25) (layer "F.Cu") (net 2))
 (segment (start 154.69 86.55) (end 152.275 88.965) (width 0.25) (layer "F.Cu") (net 2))
 (segment (start 154.99 85) (end 155.04 85.05) (width 0.25) (layer "F.Cu") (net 23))
 (segment (start 131.35 80.35) (end 131.5 80.5) (width 0.25) (layer "F.Cu") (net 23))
 (segment (start 153 85) (end 154.99 85) (width 0.25) (layer "F.Cu") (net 23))
 (segment (start 129.045 80.35) (end 131.35 80.35) (width 0.25) (layer "F.Cu") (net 23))
 (via blind (at 153 85) (size 0.8) (drill 0.4) (layers "F.Cu" "B.Cu") (free) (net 23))
 (via blind (at 131.5 80.5) (size 0.8) (drill 0.4) (layers "F.Cu" "B.Cu") (free) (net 23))
 (segment (start 146.275 78.275) (end 153 85) (width 0.25) (layer "B.Cu") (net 23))
 (segment (start 133.725 78.275) (end 146.275 78.275) (width 0.25) (layer "B.Cu") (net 23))
 (segment (start 131.5 80.5) (end 133.725 78.275) (width 0.25) (layer "B.Cu") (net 23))
 (segment (start 154.99 83.5) (end 155.04 83.55) (width 0.25) (layer "F.Cu") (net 24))
 (segment (start 118.85 80.35) (end 119 80.5) (width 0.25) (layer "F.Cu") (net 24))
 (segment (start 153 83.5) (end 154.99 83.5) (width 0.25) (layer "F.Cu") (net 24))
 (segment (start 116.455 80.35) (end 118.85 80.35) (width 0.25) (layer "F.Cu") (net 24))
 (via blind (at 153 83.5) (size 0.8) (drill 0.4) (layers "F.Cu" "B.Cu") (free) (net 24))
 (via blind (at 119 80.5) (size 0.8) (drill 0.4) (layers "F.Cu" "B.Cu") (free) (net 24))
 (segment (start 153 78.5) (end 152.25 77.75) (width 0.25) (layer "B.Cu") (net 24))
 (segment (start 120 77.75) (end 120 79.5) (width 0.25) (layer "B.Cu") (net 24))
 (segment (start 152.25 77.75) (end 120 77.75) (width 0.25) (layer "B.Cu") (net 24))
 (segment (start 153 83.5) (end 153 78.5) (width 0.25) (layer "B.Cu") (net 24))
 (segment (start 120 79.5) (end 119 80.5) (width 0.25) (layer "B.Cu") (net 24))
 (segment (start 155.04 82.05) (end 158.43 82.05) (width 0.25) (layer "F.Cu") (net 18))
 (segment (start 158.43 82.05) (end 163.25 86.87) (width 0.25) (layer "F.Cu") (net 18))
 (segment (start 155.04 80.55) (end 159.47 80.55) (width 0.25) (layer "F.Cu") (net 17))
 (segment (start 159.47 80.55) (end 163.25 84.33) (width 0.25) (layer "F.Cu") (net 17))
 (segment (start 160.51 79.05) (end 163.25 81.79) (width 0.25) (layer "F.Cu") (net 16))
 (segment (start 155.04 79.05) (end 160.51 79.05) (width 0.25) (layer "F.Cu") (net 16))
 (segment (start 161.55 77.55) (end 163.25 79.25) (width 0.25) (layer "F.Cu") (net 15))
 (segment (start 155.04 77.55) (end 161.55 77.55) (width 0.25) (layer "F.Cu") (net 15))
 (segment (start 150.73025 95.98025) (end 150.75 96) (width 0.25) (layer "F.Cu") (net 8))
 (segment (start 148.60385 95.98025) (end 150.73025 95.98025) (width 0.25) (layer "F.Cu") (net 8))
 (segment (start 116.5 105.3) (end 116.5 103.5) (width 0.25) (layer "F.Cu") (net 8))
 (via blind (at 116.5 103.5) (size 0.8) (drill 0.4) (layers "F.Cu" "B.Cu") (free) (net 8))
 (via blind (at 150.75 96) (size 0.8) (drill 0.4) (layers "F.Cu" "B.Cu") (free) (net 8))
 (segment (start 122.5 109.5) (end 151 109.5) (width 0.25) (layer "B.Cu") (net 8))
 (segment (start 151.25 96.5) (end 150.75 96) (width 0.25) (layer "B.Cu") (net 8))
 (segment (start 116.5 103.5) (end 122.5 109.5) (width 0.25) (layer "B.Cu") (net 8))
 (segment (start 151 109.5) (end 151.25 109.25) (width 0.25) (layer "B.Cu") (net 8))
 (segment (start 151.25 109.25) (end 151.25 96.5) (width 0.25) (layer "B.Cu") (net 8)))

